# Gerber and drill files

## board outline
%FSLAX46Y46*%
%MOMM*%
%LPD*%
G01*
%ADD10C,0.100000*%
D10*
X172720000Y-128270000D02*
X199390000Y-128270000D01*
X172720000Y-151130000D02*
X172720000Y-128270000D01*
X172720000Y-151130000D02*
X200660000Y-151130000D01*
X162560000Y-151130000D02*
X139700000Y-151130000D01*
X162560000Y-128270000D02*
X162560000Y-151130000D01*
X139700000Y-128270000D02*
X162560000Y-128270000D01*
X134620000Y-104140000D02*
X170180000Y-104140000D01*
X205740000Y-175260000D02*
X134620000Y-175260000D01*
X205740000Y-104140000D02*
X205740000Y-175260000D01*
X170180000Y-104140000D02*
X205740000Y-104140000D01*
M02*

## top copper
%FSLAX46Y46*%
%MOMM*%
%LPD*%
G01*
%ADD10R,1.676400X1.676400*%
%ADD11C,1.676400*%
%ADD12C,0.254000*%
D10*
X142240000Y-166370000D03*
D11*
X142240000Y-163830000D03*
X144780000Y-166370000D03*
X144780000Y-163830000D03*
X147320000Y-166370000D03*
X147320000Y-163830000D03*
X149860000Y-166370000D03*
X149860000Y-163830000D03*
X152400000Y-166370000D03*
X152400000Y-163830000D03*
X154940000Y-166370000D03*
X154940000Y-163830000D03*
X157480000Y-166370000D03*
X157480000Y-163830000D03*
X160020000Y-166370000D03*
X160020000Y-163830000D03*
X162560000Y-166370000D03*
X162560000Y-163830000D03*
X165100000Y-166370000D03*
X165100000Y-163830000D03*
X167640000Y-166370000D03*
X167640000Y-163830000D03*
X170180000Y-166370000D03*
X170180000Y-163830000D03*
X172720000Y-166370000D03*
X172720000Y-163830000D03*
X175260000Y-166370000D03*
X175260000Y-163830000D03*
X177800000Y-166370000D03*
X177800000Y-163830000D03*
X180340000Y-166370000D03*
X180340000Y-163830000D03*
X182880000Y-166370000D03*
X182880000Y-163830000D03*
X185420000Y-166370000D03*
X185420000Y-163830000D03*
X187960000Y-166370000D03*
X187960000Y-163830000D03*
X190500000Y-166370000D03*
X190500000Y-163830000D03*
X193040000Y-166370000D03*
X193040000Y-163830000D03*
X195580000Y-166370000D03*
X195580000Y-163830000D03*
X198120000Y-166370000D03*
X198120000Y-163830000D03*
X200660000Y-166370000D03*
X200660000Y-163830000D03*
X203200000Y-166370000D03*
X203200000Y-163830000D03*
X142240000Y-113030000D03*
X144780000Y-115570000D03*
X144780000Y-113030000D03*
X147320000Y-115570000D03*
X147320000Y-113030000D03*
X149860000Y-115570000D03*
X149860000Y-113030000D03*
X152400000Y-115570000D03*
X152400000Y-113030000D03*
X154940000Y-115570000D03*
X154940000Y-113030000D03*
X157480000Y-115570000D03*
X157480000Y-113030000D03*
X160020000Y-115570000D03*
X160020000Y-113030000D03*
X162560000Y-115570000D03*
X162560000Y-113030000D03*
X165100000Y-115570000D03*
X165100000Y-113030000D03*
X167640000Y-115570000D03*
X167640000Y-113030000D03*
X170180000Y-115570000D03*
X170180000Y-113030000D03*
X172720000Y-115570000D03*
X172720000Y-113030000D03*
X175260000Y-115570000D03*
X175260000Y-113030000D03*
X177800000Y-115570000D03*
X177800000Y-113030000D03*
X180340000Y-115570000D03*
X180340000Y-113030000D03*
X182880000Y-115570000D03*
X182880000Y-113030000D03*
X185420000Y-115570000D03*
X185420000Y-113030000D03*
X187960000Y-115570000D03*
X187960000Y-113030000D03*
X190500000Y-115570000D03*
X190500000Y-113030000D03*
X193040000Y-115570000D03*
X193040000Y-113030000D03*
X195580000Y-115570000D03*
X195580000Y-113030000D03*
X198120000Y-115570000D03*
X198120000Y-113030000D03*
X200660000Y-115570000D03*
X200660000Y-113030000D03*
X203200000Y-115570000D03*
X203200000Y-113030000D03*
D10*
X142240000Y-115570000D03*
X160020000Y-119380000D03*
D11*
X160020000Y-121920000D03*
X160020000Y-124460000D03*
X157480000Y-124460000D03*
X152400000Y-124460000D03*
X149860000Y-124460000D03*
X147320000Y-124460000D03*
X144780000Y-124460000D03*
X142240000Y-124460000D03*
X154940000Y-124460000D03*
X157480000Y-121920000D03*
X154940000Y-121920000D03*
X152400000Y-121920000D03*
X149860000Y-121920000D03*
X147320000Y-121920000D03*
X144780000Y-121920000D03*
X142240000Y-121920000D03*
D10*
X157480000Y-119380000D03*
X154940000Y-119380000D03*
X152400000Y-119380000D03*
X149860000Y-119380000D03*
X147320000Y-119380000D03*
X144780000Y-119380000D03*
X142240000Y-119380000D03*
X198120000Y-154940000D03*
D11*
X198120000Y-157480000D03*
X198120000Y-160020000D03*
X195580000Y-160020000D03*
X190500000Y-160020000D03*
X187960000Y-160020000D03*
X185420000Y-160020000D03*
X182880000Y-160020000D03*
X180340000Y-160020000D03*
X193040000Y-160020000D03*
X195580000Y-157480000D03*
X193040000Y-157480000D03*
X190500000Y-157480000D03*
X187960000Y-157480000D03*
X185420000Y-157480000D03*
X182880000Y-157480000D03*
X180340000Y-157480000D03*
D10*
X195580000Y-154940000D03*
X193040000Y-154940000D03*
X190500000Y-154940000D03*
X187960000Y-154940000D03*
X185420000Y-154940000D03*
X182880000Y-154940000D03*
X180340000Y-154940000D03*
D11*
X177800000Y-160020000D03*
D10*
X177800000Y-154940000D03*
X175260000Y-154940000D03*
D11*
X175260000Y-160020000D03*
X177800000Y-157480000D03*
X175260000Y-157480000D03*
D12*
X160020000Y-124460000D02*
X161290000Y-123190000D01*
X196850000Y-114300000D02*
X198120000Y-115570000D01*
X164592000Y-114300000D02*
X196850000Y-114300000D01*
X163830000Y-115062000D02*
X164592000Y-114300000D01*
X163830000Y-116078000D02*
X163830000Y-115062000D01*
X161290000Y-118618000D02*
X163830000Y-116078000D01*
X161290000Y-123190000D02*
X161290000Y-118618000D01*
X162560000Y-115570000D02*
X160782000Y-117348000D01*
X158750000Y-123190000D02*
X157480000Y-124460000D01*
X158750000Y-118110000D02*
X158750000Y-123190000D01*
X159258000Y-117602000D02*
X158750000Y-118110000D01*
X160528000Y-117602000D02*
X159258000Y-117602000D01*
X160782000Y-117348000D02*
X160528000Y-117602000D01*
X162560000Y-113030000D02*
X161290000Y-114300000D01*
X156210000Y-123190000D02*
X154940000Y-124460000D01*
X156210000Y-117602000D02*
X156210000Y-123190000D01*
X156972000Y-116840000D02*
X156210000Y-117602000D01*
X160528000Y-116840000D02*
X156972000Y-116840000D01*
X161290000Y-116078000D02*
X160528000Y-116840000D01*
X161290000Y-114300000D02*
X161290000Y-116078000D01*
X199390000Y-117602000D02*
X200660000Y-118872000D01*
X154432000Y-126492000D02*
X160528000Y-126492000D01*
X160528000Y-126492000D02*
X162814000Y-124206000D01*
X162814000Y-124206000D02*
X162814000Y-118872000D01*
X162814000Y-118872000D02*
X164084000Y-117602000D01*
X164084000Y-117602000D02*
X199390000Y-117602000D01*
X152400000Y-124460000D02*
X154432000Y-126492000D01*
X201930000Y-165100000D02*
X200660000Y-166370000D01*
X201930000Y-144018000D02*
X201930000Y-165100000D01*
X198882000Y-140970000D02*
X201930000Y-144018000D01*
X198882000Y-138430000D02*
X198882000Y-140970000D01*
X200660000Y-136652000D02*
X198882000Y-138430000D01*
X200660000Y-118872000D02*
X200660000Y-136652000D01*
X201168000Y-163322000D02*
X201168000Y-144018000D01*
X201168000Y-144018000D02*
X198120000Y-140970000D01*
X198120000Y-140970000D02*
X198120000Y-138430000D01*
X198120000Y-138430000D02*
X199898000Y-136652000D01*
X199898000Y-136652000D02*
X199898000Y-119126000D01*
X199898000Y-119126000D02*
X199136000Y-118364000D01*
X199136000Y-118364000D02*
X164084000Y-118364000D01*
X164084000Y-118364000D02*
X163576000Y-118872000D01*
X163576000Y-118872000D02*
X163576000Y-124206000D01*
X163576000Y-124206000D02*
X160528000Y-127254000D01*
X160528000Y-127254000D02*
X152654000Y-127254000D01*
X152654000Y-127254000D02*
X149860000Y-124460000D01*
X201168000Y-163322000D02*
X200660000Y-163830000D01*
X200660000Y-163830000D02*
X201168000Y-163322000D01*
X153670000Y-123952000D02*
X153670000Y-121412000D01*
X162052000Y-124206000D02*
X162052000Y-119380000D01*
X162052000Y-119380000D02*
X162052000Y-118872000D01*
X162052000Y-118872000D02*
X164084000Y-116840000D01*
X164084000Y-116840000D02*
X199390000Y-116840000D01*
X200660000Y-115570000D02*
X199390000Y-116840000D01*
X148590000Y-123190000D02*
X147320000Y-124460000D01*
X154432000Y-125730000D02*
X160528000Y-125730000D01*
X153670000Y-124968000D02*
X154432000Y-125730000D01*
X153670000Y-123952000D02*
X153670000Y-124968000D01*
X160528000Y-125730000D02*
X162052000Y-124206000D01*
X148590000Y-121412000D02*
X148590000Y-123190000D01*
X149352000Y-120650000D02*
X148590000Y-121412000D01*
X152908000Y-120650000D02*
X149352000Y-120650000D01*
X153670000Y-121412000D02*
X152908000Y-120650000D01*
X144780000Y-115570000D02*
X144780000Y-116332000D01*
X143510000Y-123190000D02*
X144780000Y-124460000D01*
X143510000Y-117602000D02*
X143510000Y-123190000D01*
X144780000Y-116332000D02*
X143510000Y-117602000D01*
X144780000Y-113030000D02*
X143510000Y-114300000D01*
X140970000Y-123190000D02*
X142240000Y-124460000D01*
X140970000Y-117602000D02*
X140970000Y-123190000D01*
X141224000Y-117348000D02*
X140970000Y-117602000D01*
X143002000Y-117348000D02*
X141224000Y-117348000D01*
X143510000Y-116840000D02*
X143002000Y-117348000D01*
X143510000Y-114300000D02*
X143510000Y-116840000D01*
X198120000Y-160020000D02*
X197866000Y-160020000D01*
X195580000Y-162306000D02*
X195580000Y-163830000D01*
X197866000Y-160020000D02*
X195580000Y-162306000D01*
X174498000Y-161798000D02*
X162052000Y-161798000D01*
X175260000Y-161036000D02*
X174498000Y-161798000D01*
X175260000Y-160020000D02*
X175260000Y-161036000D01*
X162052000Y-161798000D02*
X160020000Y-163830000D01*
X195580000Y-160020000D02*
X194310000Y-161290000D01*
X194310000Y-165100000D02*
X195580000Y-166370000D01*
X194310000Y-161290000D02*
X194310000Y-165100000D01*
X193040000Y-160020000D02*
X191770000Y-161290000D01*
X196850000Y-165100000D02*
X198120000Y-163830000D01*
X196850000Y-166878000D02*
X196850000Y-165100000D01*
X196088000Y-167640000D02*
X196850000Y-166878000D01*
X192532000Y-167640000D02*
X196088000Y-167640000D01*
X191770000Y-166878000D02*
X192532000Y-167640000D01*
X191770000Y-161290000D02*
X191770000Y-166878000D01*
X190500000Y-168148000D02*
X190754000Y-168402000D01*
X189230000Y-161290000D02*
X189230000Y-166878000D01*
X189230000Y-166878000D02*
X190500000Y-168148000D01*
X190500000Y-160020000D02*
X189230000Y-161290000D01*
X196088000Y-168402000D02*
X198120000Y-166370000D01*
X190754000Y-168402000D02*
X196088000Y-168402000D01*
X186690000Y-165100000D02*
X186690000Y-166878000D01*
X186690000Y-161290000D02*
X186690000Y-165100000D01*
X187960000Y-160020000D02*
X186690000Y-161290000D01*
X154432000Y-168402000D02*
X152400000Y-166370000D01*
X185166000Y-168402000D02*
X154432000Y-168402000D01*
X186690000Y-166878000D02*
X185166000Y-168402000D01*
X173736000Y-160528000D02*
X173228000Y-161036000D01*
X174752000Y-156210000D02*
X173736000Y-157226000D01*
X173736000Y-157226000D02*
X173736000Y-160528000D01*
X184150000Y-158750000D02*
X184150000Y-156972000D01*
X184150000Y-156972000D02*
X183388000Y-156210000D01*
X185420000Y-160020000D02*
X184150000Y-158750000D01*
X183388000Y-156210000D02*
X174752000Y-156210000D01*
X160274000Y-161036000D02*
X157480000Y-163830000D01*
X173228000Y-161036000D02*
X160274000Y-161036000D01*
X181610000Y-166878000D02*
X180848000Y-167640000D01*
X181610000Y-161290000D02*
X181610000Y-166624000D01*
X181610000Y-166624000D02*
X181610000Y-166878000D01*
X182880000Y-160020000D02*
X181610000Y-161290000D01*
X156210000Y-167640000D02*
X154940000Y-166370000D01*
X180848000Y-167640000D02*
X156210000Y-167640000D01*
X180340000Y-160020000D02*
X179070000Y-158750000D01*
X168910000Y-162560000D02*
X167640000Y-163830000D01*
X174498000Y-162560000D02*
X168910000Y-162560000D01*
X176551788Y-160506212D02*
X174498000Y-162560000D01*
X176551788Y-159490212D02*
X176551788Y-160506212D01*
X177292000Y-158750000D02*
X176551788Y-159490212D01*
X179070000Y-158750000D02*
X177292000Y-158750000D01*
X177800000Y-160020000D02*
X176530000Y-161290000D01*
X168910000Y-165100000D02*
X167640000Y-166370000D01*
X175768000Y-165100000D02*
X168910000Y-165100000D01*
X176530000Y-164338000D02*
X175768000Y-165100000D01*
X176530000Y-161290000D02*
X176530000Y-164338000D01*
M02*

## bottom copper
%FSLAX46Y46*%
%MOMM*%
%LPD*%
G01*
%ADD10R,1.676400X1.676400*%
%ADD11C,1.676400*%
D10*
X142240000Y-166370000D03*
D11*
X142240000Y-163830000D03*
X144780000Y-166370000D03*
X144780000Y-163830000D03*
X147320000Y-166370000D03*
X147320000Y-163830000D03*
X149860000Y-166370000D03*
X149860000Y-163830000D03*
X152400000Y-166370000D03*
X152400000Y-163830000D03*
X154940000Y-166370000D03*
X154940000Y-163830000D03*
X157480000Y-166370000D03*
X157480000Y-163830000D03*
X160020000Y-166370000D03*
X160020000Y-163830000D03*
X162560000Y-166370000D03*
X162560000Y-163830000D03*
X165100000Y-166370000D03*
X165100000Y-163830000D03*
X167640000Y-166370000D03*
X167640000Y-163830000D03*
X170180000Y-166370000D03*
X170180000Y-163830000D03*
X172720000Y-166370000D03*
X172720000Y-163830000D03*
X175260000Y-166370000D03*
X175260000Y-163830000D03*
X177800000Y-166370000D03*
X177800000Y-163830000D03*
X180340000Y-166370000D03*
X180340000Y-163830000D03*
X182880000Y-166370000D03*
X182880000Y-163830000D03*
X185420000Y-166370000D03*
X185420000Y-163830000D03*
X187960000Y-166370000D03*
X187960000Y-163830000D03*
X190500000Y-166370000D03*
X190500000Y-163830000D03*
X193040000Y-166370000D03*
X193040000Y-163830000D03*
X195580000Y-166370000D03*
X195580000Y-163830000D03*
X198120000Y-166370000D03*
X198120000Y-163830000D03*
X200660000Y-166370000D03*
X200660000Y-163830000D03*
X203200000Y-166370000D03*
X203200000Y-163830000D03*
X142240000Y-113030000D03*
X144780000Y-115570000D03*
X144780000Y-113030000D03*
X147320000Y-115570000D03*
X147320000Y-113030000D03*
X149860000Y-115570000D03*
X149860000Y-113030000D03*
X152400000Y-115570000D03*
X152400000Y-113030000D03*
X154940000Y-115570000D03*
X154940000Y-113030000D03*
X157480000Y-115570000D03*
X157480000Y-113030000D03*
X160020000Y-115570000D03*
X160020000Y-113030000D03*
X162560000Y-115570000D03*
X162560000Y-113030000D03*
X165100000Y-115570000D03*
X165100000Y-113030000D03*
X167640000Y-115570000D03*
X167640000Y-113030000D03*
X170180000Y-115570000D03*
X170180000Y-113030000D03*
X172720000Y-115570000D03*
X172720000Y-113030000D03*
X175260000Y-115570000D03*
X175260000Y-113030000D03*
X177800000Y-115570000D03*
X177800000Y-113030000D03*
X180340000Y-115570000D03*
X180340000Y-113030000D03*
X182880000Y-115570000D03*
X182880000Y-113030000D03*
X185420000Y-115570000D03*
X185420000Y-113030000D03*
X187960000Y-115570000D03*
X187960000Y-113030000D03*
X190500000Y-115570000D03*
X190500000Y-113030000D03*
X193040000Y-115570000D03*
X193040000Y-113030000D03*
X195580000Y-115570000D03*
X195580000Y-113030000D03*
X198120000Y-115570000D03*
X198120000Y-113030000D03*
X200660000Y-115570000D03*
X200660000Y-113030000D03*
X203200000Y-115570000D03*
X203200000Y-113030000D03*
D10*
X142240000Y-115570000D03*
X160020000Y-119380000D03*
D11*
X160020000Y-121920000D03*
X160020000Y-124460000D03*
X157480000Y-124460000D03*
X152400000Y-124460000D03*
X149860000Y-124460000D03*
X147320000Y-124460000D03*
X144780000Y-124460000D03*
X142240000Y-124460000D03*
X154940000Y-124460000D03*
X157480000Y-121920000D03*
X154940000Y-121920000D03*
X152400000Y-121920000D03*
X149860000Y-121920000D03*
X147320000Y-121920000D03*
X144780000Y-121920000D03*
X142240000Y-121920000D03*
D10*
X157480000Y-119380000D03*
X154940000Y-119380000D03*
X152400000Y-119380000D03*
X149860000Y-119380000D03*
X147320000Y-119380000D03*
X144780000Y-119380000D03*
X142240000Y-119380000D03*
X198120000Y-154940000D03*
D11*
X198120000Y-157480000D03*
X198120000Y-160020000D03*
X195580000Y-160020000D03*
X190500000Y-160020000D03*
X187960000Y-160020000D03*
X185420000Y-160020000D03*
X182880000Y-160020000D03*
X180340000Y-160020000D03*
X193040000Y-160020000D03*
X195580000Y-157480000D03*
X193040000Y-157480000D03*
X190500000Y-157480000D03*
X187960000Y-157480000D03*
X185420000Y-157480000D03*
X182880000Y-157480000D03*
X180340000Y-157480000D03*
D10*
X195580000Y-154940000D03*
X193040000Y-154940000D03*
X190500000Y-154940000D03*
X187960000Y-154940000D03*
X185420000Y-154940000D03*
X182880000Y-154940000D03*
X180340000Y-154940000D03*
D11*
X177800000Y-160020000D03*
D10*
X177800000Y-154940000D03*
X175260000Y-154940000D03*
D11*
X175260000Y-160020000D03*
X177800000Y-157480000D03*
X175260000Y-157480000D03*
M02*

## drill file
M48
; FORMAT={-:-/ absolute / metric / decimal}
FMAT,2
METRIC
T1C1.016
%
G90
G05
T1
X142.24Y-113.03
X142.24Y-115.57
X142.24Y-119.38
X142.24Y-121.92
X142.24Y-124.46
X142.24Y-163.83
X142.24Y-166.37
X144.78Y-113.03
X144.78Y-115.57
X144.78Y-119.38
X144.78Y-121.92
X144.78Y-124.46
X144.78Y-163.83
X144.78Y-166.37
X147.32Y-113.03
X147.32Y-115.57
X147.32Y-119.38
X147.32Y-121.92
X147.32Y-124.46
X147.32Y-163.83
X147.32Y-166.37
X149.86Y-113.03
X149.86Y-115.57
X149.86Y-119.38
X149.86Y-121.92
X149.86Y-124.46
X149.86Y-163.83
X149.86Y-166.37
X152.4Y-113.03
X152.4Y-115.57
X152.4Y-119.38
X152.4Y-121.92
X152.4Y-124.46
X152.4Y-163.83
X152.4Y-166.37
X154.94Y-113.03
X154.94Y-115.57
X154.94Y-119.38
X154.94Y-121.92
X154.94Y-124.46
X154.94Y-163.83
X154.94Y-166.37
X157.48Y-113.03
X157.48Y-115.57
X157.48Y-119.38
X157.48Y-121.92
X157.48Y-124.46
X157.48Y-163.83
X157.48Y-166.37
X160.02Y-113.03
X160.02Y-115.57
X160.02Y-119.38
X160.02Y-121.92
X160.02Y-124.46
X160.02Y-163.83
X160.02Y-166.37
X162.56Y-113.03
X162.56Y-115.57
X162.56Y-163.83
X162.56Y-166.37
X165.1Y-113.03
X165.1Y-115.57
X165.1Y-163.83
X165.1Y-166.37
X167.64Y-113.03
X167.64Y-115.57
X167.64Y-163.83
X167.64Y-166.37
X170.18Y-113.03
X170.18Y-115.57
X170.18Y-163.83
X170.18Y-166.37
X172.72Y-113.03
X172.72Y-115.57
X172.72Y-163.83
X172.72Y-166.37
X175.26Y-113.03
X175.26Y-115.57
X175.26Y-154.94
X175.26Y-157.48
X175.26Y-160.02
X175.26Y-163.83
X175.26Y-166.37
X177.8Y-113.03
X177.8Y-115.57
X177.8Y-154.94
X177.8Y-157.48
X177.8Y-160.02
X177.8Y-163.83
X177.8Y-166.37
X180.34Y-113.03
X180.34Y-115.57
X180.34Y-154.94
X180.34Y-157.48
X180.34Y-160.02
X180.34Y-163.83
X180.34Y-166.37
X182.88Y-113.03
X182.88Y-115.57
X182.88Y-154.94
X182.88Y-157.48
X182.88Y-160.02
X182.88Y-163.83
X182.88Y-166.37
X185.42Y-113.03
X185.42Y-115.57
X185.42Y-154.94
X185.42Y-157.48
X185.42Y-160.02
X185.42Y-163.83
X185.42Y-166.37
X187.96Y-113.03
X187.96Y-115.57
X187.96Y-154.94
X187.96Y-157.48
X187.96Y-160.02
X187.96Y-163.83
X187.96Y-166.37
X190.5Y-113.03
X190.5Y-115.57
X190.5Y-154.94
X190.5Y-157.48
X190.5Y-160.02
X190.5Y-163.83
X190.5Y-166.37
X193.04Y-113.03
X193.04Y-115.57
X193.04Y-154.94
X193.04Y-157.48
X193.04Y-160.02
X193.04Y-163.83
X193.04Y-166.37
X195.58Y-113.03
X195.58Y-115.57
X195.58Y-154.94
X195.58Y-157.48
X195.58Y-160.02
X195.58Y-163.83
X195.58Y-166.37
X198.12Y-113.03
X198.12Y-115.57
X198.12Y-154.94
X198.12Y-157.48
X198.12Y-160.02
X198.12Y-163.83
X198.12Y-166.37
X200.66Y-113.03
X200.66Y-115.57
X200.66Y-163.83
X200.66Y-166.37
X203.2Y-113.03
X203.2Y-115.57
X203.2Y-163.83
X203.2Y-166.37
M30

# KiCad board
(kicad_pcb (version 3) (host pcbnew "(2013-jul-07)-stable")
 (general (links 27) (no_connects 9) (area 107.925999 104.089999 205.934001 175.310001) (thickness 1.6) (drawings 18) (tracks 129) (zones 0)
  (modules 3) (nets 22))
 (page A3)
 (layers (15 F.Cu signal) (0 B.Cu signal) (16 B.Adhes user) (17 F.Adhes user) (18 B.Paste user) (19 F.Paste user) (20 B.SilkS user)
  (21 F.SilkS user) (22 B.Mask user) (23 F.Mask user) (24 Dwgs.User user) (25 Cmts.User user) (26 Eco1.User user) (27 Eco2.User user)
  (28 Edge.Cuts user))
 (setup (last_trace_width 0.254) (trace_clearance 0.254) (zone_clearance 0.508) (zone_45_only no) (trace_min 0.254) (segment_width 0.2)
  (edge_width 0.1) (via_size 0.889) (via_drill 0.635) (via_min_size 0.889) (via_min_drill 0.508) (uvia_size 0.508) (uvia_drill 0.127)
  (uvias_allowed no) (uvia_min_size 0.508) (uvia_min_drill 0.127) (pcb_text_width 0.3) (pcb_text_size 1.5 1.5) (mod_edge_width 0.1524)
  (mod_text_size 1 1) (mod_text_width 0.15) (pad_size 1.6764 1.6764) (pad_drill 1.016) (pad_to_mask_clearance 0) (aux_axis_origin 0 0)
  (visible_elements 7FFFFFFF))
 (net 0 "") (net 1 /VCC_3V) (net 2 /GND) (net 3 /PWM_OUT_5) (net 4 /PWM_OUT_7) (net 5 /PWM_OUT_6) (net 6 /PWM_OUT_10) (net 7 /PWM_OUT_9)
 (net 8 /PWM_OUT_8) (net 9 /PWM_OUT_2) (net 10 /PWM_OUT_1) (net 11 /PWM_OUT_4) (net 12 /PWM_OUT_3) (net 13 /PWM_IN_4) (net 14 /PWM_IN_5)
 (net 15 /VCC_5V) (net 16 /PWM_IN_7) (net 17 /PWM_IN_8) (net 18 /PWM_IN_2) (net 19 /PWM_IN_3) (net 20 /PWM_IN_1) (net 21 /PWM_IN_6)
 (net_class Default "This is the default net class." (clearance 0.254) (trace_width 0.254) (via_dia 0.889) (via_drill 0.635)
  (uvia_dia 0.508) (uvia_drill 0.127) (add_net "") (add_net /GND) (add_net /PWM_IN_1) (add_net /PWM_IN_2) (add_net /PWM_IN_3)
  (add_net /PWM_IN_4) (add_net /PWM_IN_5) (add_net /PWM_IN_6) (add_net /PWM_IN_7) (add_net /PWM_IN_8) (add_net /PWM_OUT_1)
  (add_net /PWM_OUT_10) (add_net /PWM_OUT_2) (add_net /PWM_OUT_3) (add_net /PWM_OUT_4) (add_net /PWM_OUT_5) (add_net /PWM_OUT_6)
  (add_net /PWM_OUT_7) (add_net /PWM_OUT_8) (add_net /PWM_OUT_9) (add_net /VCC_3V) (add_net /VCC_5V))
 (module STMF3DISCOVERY (layer F.Cu) (at 172.72 139.7)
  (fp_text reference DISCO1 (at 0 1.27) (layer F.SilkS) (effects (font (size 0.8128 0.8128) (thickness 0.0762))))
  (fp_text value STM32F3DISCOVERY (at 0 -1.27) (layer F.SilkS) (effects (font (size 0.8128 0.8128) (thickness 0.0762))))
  (pad 6 thru_hole rect (at -30.48 26.67) (size 1.6764 1.6764) (drill 1.016) (layers *.Cu *.Mask F.SilkS) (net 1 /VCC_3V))
  (pad 20 thru_hole circle (at -30.48 24.13) (size 1.6764 1.6764) (drill 1.016) (layers *.Cu *.Mask F.SilkS) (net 1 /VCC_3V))
  (pad 49 thru_hole circle (at -27.94 26.67) (size 1.6764 1.6764) (drill 1.016) (layers *.Cu *.Mask F.SilkS) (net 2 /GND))
  (pad 14 thru_hole circle (at -27.94 24.13) (size 1.6764 1.6764) (drill 1.016) (layers *.Cu *.Mask F.SilkS))
  (pad 16 thru_hole circle (at -25.4 26.67) (size 1.6764 1.6764) (drill 1.016) (layers *.Cu *.Mask F.SilkS))
  (pad 15 thru_hole circle (at -25.4 24.13) (size 1.6764 1.6764) (drill 1.016) (layers *.Cu *.Mask F.SilkS))
  (pad 18 thru_hole circle (at -22.86 26.67) (size 1.6764 1.6764) (drill 1.016) (layers *.Cu *.Mask F.SilkS))
  (pad 17 thru_hole circle (at -22.86 24.13) (size 1.6764 1.6764) (drill 1.016) (layers *.Cu *.Mask F.SilkS))
  (pad 24 thru_hole circle (at -20.32 26.67) (size 1.6764 1.6764) (drill 1.016) (layers *.Cu *.Mask F.SilkS) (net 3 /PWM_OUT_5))
  (pad 19 thru_hole circle (at -20.32 24.13) (size 1.6764 1.6764) (drill 1.016) (layers *.Cu *.Mask F.SilkS))
  (pad 26 thru_hole circle (at -17.78 26.67) (size 1.6764 1.6764) (drill 1.016) (layers *.Cu *.Mask F.SilkS) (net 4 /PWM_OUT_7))
  (pad 23 thru_hole circle (at -17.78 24.13) (size 1.6764 1.6764) (drill 1.016) (layers *.Cu *.Mask F.SilkS))
  (pad 27 thru_hole circle (at -15.24 26.67) (size 1.6764 1.6764) (drill 1.016) (layers *.Cu *.Mask F.SilkS))
  (pad 25 thru_hole circle (at -15.24 24.13) (size 1.6764 1.6764) (drill 1.016) (layers *.Cu *.Mask F.SilkS) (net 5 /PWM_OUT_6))
  (pad 30 thru_hole circle (at -12.7 26.67) (size 1.6764 1.6764) (drill 1.016) (layers *.Cu *.Mask F.SilkS))
  (pad 29 thru_hole circle (at -12.7 24.13) (size 1.6764 1.6764) (drill 1.016) (layers *.Cu *.Mask F.SilkS) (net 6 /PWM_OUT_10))
  (pad 32 thru_hole circle (at -10.16 26.67) (size 1.6764 1.6764) (drill 1.016) (layers *.Cu *.Mask F.SilkS))
  (pad 31 thru_hole circle (at -10.16 24.13) (size 1.6764 1.6764) (drill 1.016) (layers *.Cu *.Mask F.SilkS))
  (pad 34 thru_hole circle (at -7.62 26.67) (size 1.6764 1.6764) (drill 1.016) (layers *.Cu *.Mask F.SilkS))
  (pad 33 thru_hole circle (at -7.62 24.13) (size 1.6764 1.6764) (drill 1.016) (layers *.Cu *.Mask F.SilkS))
  (pad 36 thru_hole circle (at -5.08 26.67) (size 1.6764 1.6764) (drill 1.016) (layers *.Cu *.Mask F.SilkS) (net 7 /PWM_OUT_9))
  (pad 35 thru_hole circle (at -5.08 24.13) (size 1.6764 1.6764) (drill 1.016) (layers *.Cu *.Mask F.SilkS) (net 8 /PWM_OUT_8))
  (pad 38 thru_hole circle (at -2.54 26.67) (size 1.6764 1.6764) (drill 1.016) (layers *.Cu *.Mask F.SilkS))
  (pad 37 thru_hole circle (at -2.54 24.13) (size 1.6764 1.6764) (drill 1.016) (layers *.Cu *.Mask F.SilkS))
  (pad 40 thru_hole circle (at 0 26.67) (size 1.6764 1.6764) (drill 1.016) (layers *.Cu *.Mask F.SilkS))
  (pad 39 thru_hole circle (at 0 24.13) (size 1.6764 1.6764) (drill 1.016) (layers *.Cu *.Mask F.SilkS))
  (pad 42 thru_hole circle (at 2.54 26.67) (size 1.6764 1.6764) (drill 1.016) (layers *.Cu *.Mask F.SilkS))
  (pad 41 thru_hole circle (at 2.54 24.13) (size 1.6764 1.6764) (drill 1.016) (layers *.Cu *.Mask F.SilkS))
  (pad 44 thru_hole circle (at 5.08 26.67) (size 1.6764 1.6764) (drill 1.016) (layers *.Cu *.Mask F.SilkS))
  (pad 43 thru_hole circle (at 5.08 24.13) (size 1.6764 1.6764) (drill 1.016) (layers *.Cu *.Mask F.SilkS))
  (pad 46 thru_hole circle (at 7.62 26.67) (size 1.6764 1.6764) (drill 1.016) (layers *.Cu *.Mask F.SilkS))
  (pad 45 thru_hole circle (at 7.62 24.13) (size 1.6764 1.6764) (drill 1.016) (layers *.Cu *.Mask F.SilkS))
  (pad 48 thru_hole circle (at 10.16 26.67) (size 1.6764 1.6764) (drill 1.016) (layers *.Cu *.Mask F.SilkS))
  (pad 47 thru_hole circle (at 10.16 24.13) (size 1.6764 1.6764) (drill 1.016) (layers *.Cu *.Mask F.SilkS))
  (pad 52 thru_hole circle (at 12.7 26.67) (size 1.6764 1.6764) (drill 1.016) (layers *.Cu *.Mask F.SilkS))
  (pad 51 thru_hole circle (at 12.7 24.13) (size 1.6764 1.6764) (drill 1.016) (layers *.Cu *.Mask F.SilkS))
  (pad 54 thru_hole circle (at 15.24 26.67) (size 1.6764 1.6764) (drill 1.016) (layers *.Cu *.Mask F.SilkS))
  (pad 53 thru_hole circle (at 15.24 24.13) (size 1.6764 1.6764) (drill 1.016) (layers *.Cu *.Mask F.SilkS))
  (pad 56 thru_hole circle (at 17.78 26.67) (size 1.6764 1.6764) (drill 1.016) (layers *.Cu *.Mask F.SilkS))
  (pad 55 thru_hole circle (at 17.78 24.13) (size 1.6764 1.6764) (drill 1.016) (layers *.Cu *.Mask F.SilkS))
  (pad 58 thru_hole circle (at 20.32 26.67) (size 1.6764 1.6764) (drill 1.016) (layers *.Cu *.Mask F.SilkS))
  (pad 57 thru_hole circle (at 20.32 24.13) (size 1.6764 1.6764) (drill 1.016) (layers *.Cu *.Mask F.SilkS))
  (pad 60 thru_hole circle (at 22.86 26.67) (size 1.6764 1.6764) (drill 1.016) (layers *.Cu *.Mask F.SilkS) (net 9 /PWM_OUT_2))
  (pad 59 thru_hole circle (at 22.86 24.13) (size 1.6764 1.6764) (drill 1.016) (layers *.Cu *.Mask F.SilkS) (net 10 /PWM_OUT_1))
  (pad 62 thru_hole circle (at 25.4 26.67) (size 1.6764 1.6764) (drill 1.016) (layers *.Cu *.Mask F.SilkS) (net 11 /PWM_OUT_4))
  (pad 61 thru_hole circle (at 25.4 24.13) (size 1.6764 1.6764) (drill 1.016) (layers *.Cu *.Mask F.SilkS) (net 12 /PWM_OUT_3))
  (pad 63 thru_hole circle (at 27.94 26.67) (size 1.6764 1.6764) (drill 1.016) (layers *.Cu *.Mask F.SilkS) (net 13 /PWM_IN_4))
  (pad 64 thru_hole circle (at 27.94 24.13) (size 1.6764 1.6764) (drill 1.016) (layers *.Cu *.Mask F.SilkS) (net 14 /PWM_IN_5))
  (pad 50 thru_hole circle (at 30.48 26.67) (size 1.6764 1.6764) (drill 1.016) (layers *.Cu *.Mask F.SilkS) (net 2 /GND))
  (pad 74 thru_hole circle (at 30.48 24.13) (size 1.6764 1.6764) (drill 1.016) (layers *.Cu *.Mask F.SilkS) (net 2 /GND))
  (pad 22 thru_hole circle (at -30.48 -26.67) (size 1.6764 1.6764) (drill 1.016) (layers *.Cu *.Mask F.SilkS) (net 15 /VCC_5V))
  (pad 10 thru_hole circle (at -27.94 -24.13) (size 1.6764 1.6764) (drill 1.016) (layers *.Cu *.Mask F.SilkS) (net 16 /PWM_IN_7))
  (pad 11 thru_hole circle (at -27.94 -26.67) (size 1.6764 1.6764) (drill 1.016) (layers *.Cu *.Mask F.SilkS) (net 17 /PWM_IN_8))
  (pad 12 thru_hole circle (at -25.4 -24.13) (size 1.6764 1.6764) (drill 1.016) (layers *.Cu *.Mask F.SilkS))
  (pad 13 thru_hole circle (at -25.4 -26.67) (size 1.6764 1.6764) (drill 1.016) (layers *.Cu *.Mask F.SilkS))
  (pad 8 thru_hole circle (at -22.86 -24.13) (size 1.6764 1.6764) (drill 1.016) (layers *.Cu *.Mask F.SilkS))
  (pad 9 thru_hole circle (at -22.86 -26.67) (size 1.6764 1.6764) (drill 1.016) (layers *.Cu *.Mask F.SilkS))
  (pad 5 thru_hole circle (at -20.32 -24.13) (size 1.6764 1.6764) (drill 1.016) (layers *.Cu *.Mask F.SilkS))
  (pad 7 thru_hole circle (at -20.32 -26.67) (size 1.6764 1.6764) (drill 1.016) (layers *.Cu *.Mask F.SilkS))
  (pad 3 thru_hole circle (at -17.78 -24.13) (size 1.6764 1.6764) (drill 1.016) (layers *.Cu *.Mask F.SilkS))
  (pad 4 thru_hole circle (at -17.78 -26.67) (size 1.6764 1.6764) (drill 1.016) (layers *.Cu *.Mask F.SilkS))
  (pad 1 thru_hole circle (at -15.24 -24.13) (size 1.6764 1.6764) (drill 1.016) (layers *.Cu *.Mask F.SilkS))
  (pad 2 thru_hole circle (at -15.24 -26.67) (size 1.6764 1.6764) (drill 1.016) (layers *.Cu *.Mask F.SilkS))
  (pad 97 thru_hole circle (at -12.7 -24.13) (size 1.6764 1.6764) (drill 1.016) (layers *.Cu *.Mask F.SilkS))
  (pad 98 thru_hole circle (at -12.7 -26.67) (size 1.6764 1.6764) (drill 1.016) (layers *.Cu *.Mask F.SilkS))
  (pad 95 thru_hole circle (at -10.16 -24.13) (size 1.6764 1.6764) (drill 1.016) (layers *.Cu *.Mask F.SilkS) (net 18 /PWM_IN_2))
  (pad 96 thru_hole circle (at -10.16 -26.67) (size 1.6764 1.6764) (drill 1.016) (layers *.Cu *.Mask F.SilkS) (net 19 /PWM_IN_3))
  (pad 94 thru_hole circle (at -7.62 -24.13) (size 1.6764 1.6764) (drill 1.016) (layers *.Cu *.Mask F.SilkS))
  (pad 28 thru_hole circle (at -7.62 -26.67) (size 1.6764 1.6764) (drill 1.016) (layers *.Cu *.Mask F.SilkS))
  (pad 92 thru_hole circle (at -5.08 -24.13) (size 1.6764 1.6764) (drill 1.016) (layers *.Cu *.Mask F.SilkS))
  (pad 93 thru_hole circle (at -5.08 -26.67) (size 1.6764 1.6764) (drill 1.016) (layers *.Cu *.Mask F.SilkS))
  (pad 90 thru_hole circle (at -2.54 -24.13) (size 1.6764 1.6764) (drill 1.016) (layers *.Cu *.Mask F.SilkS))
  (pad 91 thru_hole circle (at -2.54 -26.67) (size 1.6764 1.6764) (drill 1.016) (layers *.Cu *.Mask F.SilkS))
  (pad 88 thru_hole circle (at 0 -24.13) (size 1.6764 1.6764) (drill 1.016) (layers *.Cu *.Mask F.SilkS))
  (pad 89 thru_hole circle (at 0 -26.67) (size 1.6764 1.6764) (drill 1.016) (layers *.Cu *.Mask F.SilkS))
  (pad 86 thru_hole circle (at 2.54 -24.13) (size 1.6764 1.6764) (drill 1.016) (layers *.Cu *.Mask F.SilkS))
  (pad 87 thru_hole circle (at 2.54 -26.67) (size 1.6764 1.6764) (drill 1.016) (layers *.Cu *.Mask F.SilkS))
  (pad 84 thru_hole circle (at 5.08 -24.13) (size 1.6764 1.6764) (drill 1.016) (layers *.Cu *.Mask F.SilkS))
  (pad 85 thru_hole circle (at 5.08 -26.67) (size 1.6764 1.6764) (drill 1.016) (layers *.Cu *.Mask F.SilkS))
  (pad 82 thru_hole circle (at 7.62 -24.13) (size 1.6764 1.6764) (drill 1.016) (layers *.Cu *.Mask F.SilkS))
  (pad 83 thru_hole circle (at 7.62 -26.67) (size 1.6764 1.6764) (drill 1.016) (layers *.Cu *.Mask F.SilkS))
  (pad 80 thru_hole circle (at 10.16 -24.13) (size 1.6764 1.6764) (drill 1.016) (layers *.Cu *.Mask F.SilkS))
  (pad 81 thru_hole circle (at 10.16 -26.67) (size 1.6764 1.6764) (drill 1.016) (layers *.Cu *.Mask F.SilkS))
  (pad 78 thru_hole circle (at 12.7 -24.13) (size 1.6764 1.6764) (drill 1.016) (layers *.Cu *.Mask F.SilkS))
  (pad 79 thru_hole circle (at 12.7 -26.67) (size 1.6764 1.6764) (drill 1.016) (layers *.Cu *.Mask F.SilkS))
  (pad 76 thru_hole circle (at 15.24 -24.13) (size 1.6764 1.6764) (drill 1.016) (layers *.Cu *.Mask F.SilkS))
  (pad 77 thru_hole circle (at 15.24 -26.67) (size 1.6764 1.6764) (drill 1.016) (layers *.Cu *.Mask F.SilkS))
  (pad 73 thru_hole circle (at 17.78 -24.13) (size 1.6764 1.6764) (drill 1.016) (layers *.Cu *.Mask F.SilkS))
  (pad 72 thru_hole circle (at 17.78 -26.67) (size 1.6764 1.6764) (drill 1.016) (layers *.Cu *.Mask F.SilkS))
  (pad 71 thru_hole circle (at 20.32 -24.13) (size 1.6764 1.6764) (drill 1.016) (layers *.Cu *.Mask F.SilkS))
  (pad 70 thru_hole circle (at 20.32 -26.67) (size 1.6764 1.6764) (drill 1.016) (layers *.Cu *.Mask F.SilkS))
  (pad 69 thru_hole circle (at 22.86 -24.13) (size 1.6764 1.6764) (drill 1.016) (layers *.Cu *.Mask F.SilkS))
  (pad 68 thru_hole circle (at 22.86 -26.67) (size 1.6764 1.6764) (drill 1.016) (layers *.Cu *.Mask F.SilkS))
  (pad 67 thru_hole circle (at 25.4 -24.13) (size 1.6764 1.6764) (drill 1.016) (layers *.Cu *.Mask F.SilkS) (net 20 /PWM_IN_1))
  (pad 66 thru_hole circle (at 25.4 -26.67) (size 1.6764 1.6764) (drill 1.016) (layers *.Cu *.Mask F.SilkS))
  (pad 65 thru_hole circle (at 27.94 -24.13) (size 1.6764 1.6764) (drill 1.016) (layers *.Cu *.Mask F.SilkS) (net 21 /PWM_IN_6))
  (pad 100 thru_hole circle (at 27.94 -26.67) (size 1.6764 1.6764) (drill 1.016) (layers *.Cu *.Mask F.SilkS))
  (pad 75 thru_hole circle (at 30.48 -24.13) (size 1.6764 1.6764) (drill 1.016) (layers *.Cu *.Mask F.SilkS) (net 2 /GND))
  (pad 99 thru_hole circle (at 30.48 -26.67) (size 1.6764 1.6764) (drill 1.016) (layers *.Cu *.Mask F.SilkS) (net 2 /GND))
  (pad 21 thru_hole rect (at -30.48 -24.13) (size 1.6764 1.6764) (drill 1.016) (layers *.Cu *.Mask F.SilkS) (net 15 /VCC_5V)))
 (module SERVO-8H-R (layer F.Cu) (at 151.13 121.92 180)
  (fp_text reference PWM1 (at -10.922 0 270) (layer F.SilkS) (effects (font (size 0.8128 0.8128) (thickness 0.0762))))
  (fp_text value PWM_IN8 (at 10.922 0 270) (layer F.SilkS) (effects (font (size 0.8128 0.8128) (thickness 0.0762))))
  (pad 1 thru_hole rect (at -8.89 2.54 180) (size 1.6764 1.6764) (drill 1.016) (layers *.Cu *.Mask F.SilkS) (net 2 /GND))
  (pad 2 thru_hole circle (at -8.89 0 180) (size 1.6764 1.6764) (drill 1.016) (layers *.Cu *.Mask F.SilkS))
  (pad 3 thru_hole circle (at -8.89 -2.54 180) (size 1.6764 1.6764) (drill 1.016) (layers *.Cu *.Mask F.SilkS) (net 20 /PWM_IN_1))
  (pad 4 thru_hole circle (at -6.35 -2.54 180) (size 1.6764 1.6764) (drill 1.016) (layers *.Cu *.Mask F.SilkS) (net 18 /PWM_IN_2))
  (pad 6 thru_hole circle (at -1.27 -2.54 180) (size 1.6764 1.6764) (drill 1.016) (layers *.Cu *.Mask F.SilkS) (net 13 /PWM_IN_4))
  (pad 7 thru_hole circle (at 1.27 -2.54 180) (size 1.6764 1.6764) (drill 1.016) (layers *.Cu *.Mask F.SilkS) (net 14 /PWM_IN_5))
  (pad 8 thru_hole circle (at 3.81 -2.54 180) (size 1.6764 1.6764) (drill 1.016) (layers *.Cu *.Mask F.SilkS) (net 21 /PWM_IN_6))
  (pad 9 thru_hole circle (at 6.35 -2.54 180) (size 1.6764 1.6764) (drill 1.016) (layers *.Cu *.Mask F.SilkS) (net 16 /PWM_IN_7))
  (pad 10 thru_hole circle (at 8.89 -2.54 180) (size 1.6764 1.6764) (drill 1.016) (layers *.Cu *.Mask F.SilkS) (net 17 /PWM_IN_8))
  (pad 5 thru_hole circle (at -3.81 -2.54 180) (size 1.6764 1.6764) (drill 1.016) (layers *.Cu *.Mask F.SilkS) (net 19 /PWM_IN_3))
  (pad "" thru_hole circle (at -6.35 0 180) (size 1.6764 1.6764) (drill 1.016) (layers *.Cu *.Mask F.SilkS))
  (pad "" thru_hole circle (at -3.81 0 180) (size 1.6764 1.6764) (drill 1.016) (layers *.Cu *.Mask F.SilkS))
  (pad "" thru_hole circle (at -1.27 0 180) (size 1.6764 1.6764) (drill 1.016) (layers *.Cu *.Mask F.SilkS))
  (pad "" thru_hole circle (at 1.27 0 180) (size 1.6764 1.6764) (drill 1.016) (layers *.Cu *.Mask F.SilkS))
  (pad "" thru_hole circle (at 3.81 0 180) (size 1.6764 1.6764) (drill 1.016) (layers *.Cu *.Mask F.SilkS))
  (pad "" thru_hole circle (at 6.35 0 180) (size 1.6764 1.6764) (drill 1.016) (layers *.Cu *.Mask F.SilkS))
  (pad "" thru_hole circle (at 8.89 0 180) (size 1.6764 1.6764) (drill 1.016) (layers *.Cu *.Mask F.SilkS))
  (pad "" thru_hole rect (at -6.35 2.54 180) (size 1.6764 1.6764) (drill 1.016) (layers *.Cu *.Mask F.SilkS))
  (pad "" thru_hole rect (at -3.81 2.54 180) (size 1.6764 1.6764) (drill 1.016) (layers *.Cu *.Mask F.SilkS))
  (pad "" thru_hole rect (at -1.27 2.54 180) (size 1.6764 1.6764) (drill 1.016) (layers *.Cu *.Mask F.SilkS))
  (pad "" thru_hole rect (at 1.27 2.54 180) (size 1.6764 1.6764) (drill 1.016) (layers *.Cu *.Mask F.SilkS))
  (pad "" thru_hole rect (at 3.81 2.54 180) (size 1.6764 1.6764) (drill 1.016) (layers *.Cu *.Mask F.SilkS))
  (pad "" thru_hole rect (at 6.35 2.54 180) (size 1.6764 1.6764) (drill 1.016) (layers *.Cu *.Mask F.SilkS))
  (pad "" thru_hole rect (at 8.89 2.54 180) (size 1.6764 1.6764) (drill 1.016) (layers *.Cu *.Mask F.SilkS)))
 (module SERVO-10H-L (layer F.Cu) (at 186.69 157.48 180)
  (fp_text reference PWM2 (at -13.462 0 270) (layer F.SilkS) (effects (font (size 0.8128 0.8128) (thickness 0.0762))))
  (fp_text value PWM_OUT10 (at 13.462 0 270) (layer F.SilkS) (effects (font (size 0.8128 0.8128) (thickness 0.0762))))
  (pad 1 thru_hole rect (at -11.43 2.54 180) (size 1.6764 1.6764) (drill 1.016) (layers *.Cu *.Mask F.SilkS) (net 2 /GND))
  (pad 2 thru_hole circle (at -11.43 0 180) (size 1.6764 1.6764) (drill 1.016) (layers *.Cu *.Mask F.SilkS))
  (pad 3 thru_hole circle (at -11.43 -2.54 180) (size 1.6764 1.6764) (drill 1.016) (layers *.Cu *.Mask F.SilkS) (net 10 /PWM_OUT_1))
  (pad 4 thru_hole circle (at -8.89 -2.54 180) (size 1.6764 1.6764) (drill 1.016) (layers *.Cu *.Mask F.SilkS) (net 9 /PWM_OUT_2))
  (pad 6 thru_hole circle (at -3.81 -2.54 180) (size 1.6764 1.6764) (drill 1.016) (layers *.Cu *.Mask F.SilkS) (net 11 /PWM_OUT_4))
  (pad 7 thru_hole circle (at -1.27 -2.54 180) (size 1.6764 1.6764) (drill 1.016) (layers *.Cu *.Mask F.SilkS) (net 3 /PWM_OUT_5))
  (pad 8 thru_hole circle (at 1.27 -2.54 180) (size 1.6764 1.6764) (drill 1.016) (layers *.Cu *.Mask F.SilkS) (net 5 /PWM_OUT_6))
  (pad 9 thru_hole circle (at 3.81 -2.54 180) (size 1.6764 1.6764) (drill 1.016) (layers *.Cu *.Mask F.SilkS) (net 4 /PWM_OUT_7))
  (pad 10 thru_hole circle (at 6.35 -2.54 180) (size 1.6764 1.6764) (drill 1.016) (layers *.Cu *.Mask F.SilkS) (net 8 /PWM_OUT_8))
  (pad 5 thru_hole circle (at -6.35 -2.54 180) (size 1.6764 1.6764) (drill 1.016) (layers *.Cu *.Mask F.SilkS) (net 12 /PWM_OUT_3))
  (pad "" thru_hole circle (at -8.89 0 180) (size 1.6764 1.6764) (drill 1.016) (layers *.Cu *.Mask F.SilkS))
  (pad "" thru_hole circle (at -6.35 0 180) (size 1.6764 1.6764) (drill 1.016) (layers *.Cu *.Mask F.SilkS))
  (pad "" thru_hole circle (at -3.81 0 180) (size 1.6764 1.6764) (drill 1.016) (layers *.Cu *.Mask F.SilkS))
  (pad "" thru_hole circle (at -1.27 0 180) (size 1.6764 1.6764) (drill 1.016) (layers *.Cu *.Mask F.SilkS))
  (pad "" thru_hole circle (at 1.27 0 180) (size 1.6764 1.6764) (drill 1.016) (layers *.Cu *.Mask F.SilkS))
  (pad "" thru_hole circle (at 3.81 0 180) (size 1.6764 1.6764) (drill 1.016) (layers *.Cu *.Mask F.SilkS))
  (pad "" thru_hole circle (at 6.35 0 180) (size 1.6764 1.6764) (drill 1.016) (layers *.Cu *.Mask F.SilkS))
  (pad "" thru_hole rect (at -8.89 2.54 180) (size 1.6764 1.6764) (drill 1.016) (layers *.Cu *.Mask F.SilkS))
  (pad "" thru_hole rect (at -6.35 2.54 180) (size 1.6764 1.6764) (drill 1.016) (layers *.Cu *.Mask F.SilkS))
  (pad "" thru_hole rect (at -3.81 2.54 180) (size 1.6764 1.6764) (drill 1.016) (layers *.Cu *.Mask F.SilkS))
  (pad "" thru_hole rect (at -1.27 2.54 180) (size 1.6764 1.6764) (drill 1.016) (layers *.Cu *.Mask F.SilkS))
  (pad "" thru_hole rect (at 1.27 2.54 180) (size 1.6764 1.6764) (drill 1.016) (layers *.Cu *.Mask F.SilkS))
  (pad "" thru_hole rect (at 3.81 2.54 180) (size 1.6764 1.6764) (drill 1.016) (layers *.Cu *.Mask F.SilkS))
  (pad "" thru_hole rect (at 6.35 2.54 180) (size 1.6764 1.6764) (drill 1.016) (layers *.Cu *.Mask F.SilkS))
  (pad 11 thru_hole circle (at 8.89 -2.54 180) (size 1.6764 1.6764) (drill 1.016) (layers *.Cu *.Mask F.SilkS) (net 7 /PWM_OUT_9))
  (pad "" thru_hole rect (at 8.89 2.54 180) (size 1.6764 1.6764) (drill 1.016) (layers *.Cu *.Mask F.SilkS))
  (pad "" thru_hole rect (at 11.43 2.54 180) (size 1.6764 1.6764) (drill 1.016) (layers *.Cu *.Mask F.SilkS))
  (pad 12 thru_hole circle (at 11.43 -2.54 180) (size 1.6764 1.6764) (drill 1.016) (layers *.Cu *.Mask F.SilkS) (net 6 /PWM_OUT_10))
  (pad "" thru_hole circle (at 8.89 0 180) (size 1.6764 1.6764) (drill 1.016) (layers *.Cu *.Mask F.SilkS))
  (pad "" thru_hole circle (at 11.43 0 180) (size 1.6764 1.6764) (drill 1.016) (layers *.Cu *.Mask F.SilkS)))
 (gr_line (start 172.72 128.27) (end 199.39 128.27) (angle 90) (layer Edge.Cuts) (width 0.1))
 (gr_line (start 172.72 151.13) (end 172.72 128.27) (angle 90) (layer Edge.Cuts) (width 0.1))
 (gr_line (start 172.72 151.13) (end 200.66 151.13) (angle 90) (layer Edge.Cuts) (width 0.1))
 (gr_line (start 162.56 151.13) (end 139.7 151.13) (angle 90) (layer Edge.Cuts) (width 0.1))
 (gr_line (start 162.56 128.27) (end 162.56 151.13) (angle 90) (layer Edge.Cuts) (width 0.1))
 (gr_line (start 139.7 128.27) (end 162.56 128.27) (angle 90) (layer Edge.Cuts) (width 0.1))
 (gr_line (start 134.62 104.14) (end 170.18 104.14) (angle 90) (layer Edge.Cuts) (width 0.1))
 (gr_line (start 205.74 175.26) (end 134.62 175.26) (angle 90) (layer Edge.Cuts) (width 0.1))
 (gr_line (start 205.74 104.14) (end 205.74 175.26) (angle 90) (layer Edge.Cuts) (width 0.1))
 (gr_line (start 170.18 104.14) (end 205.74 104.14) (angle 90) (layer Edge.Cuts) (width 0.1))
 (segment (start 160.02 124.46) (end 161.29 123.19) (width 0.254) (layer F.Cu) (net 20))
 (segment (start 196.85 114.3) (end 198.12 115.57) (width 0.254) (layer F.Cu) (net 20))
 (segment (start 164.592 114.3) (end 196.85 114.3) (width 0.254) (layer F.Cu) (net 20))
 (segment (start 163.83 115.062) (end 164.592 114.3) (width 0.254) (layer F.Cu) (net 20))
 (segment (start 163.83 116.078) (end 163.83 115.062) (width 0.254) (layer F.Cu) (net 20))
 (segment (start 161.29 118.618) (end 163.83 116.078) (width 0.254) (layer F.Cu) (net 20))
 (segment (start 161.29 123.19) (end 161.29 118.618) (width 0.254) (layer F.Cu) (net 20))
 (segment (start 162.56 115.57) (end 160.782 117.348) (width 0.254) (layer F.Cu) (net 18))
 (segment (start 158.75 123.19) (end 157.48 124.46) (width 0.254) (layer F.Cu) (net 18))
 (segment (start 158.75 118.11) (end 158.75 123.19) (width 0.254) (layer F.Cu) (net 18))
 (segment (start 159.258 117.602) (end 158.75 118.11) (width 0.254) (layer F.Cu) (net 18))
 (segment (start 160.528 117.602) (end 159.258 117.602) (width 0.254) (layer F.Cu) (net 18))
 (segment (start 160.782 117.348) (end 160.528 117.602) (width 0.254) (layer F.Cu) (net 18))
 (segment (start 162.56 113.03) (end 161.29 114.3) (width 0.254) (layer F.Cu) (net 19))
 (segment (start 156.21 123.19) (end 154.94 124.46) (width 0.254) (layer F.Cu) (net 19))
 (segment (start 156.21 117.602) (end 156.21 123.19) (width 0.254) (layer F.Cu) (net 19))
 (segment (start 156.972 116.84) (end 156.21 117.602) (width 0.254) (layer F.Cu) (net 19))
 (segment (start 160.528 116.84) (end 156.972 116.84) (width 0.254) (layer F.Cu) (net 19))
 (segment (start 161.29 116.078) (end 160.528 116.84) (width 0.254) (layer F.Cu) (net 19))
 (segment (start 161.29 114.3) (end 161.29 116.078) (width 0.254) (layer F.Cu) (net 19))
 (segment (start 199.39 117.602) (end 200.66 118.872) (width 0.254) (layer F.Cu) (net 13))
 (segment (start 154.432 126.492) (end 160.528 126.492) (width 0.254) (layer F.Cu) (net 13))
 (segment (start 160.528 126.492) (end 162.814 124.206) (width 0.254) (layer F.Cu) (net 13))
 (segment (start 162.814 124.206) (end 162.814 118.872) (width 0.254) (layer F.Cu) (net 13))
 (segment (start 162.814 118.872) (end 164.084 117.602) (width 0.254) (layer F.Cu) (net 13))
 (segment (start 164.084 117.602) (end 199.39 117.602) (width 0.254) (layer F.Cu) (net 13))
 (segment (start 152.4 124.46) (end 154.432 126.492) (width 0.254) (layer F.Cu) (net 13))
 (segment (start 201.93 165.1) (end 200.66 166.37) (width 0.254) (layer F.Cu) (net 13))
 (segment (start 201.93 144.018) (end 201.93 165.1) (width 0.254) (layer F.Cu) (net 13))
 (segment (start 198.882 140.97) (end 201.93 144.018) (width 0.254) (layer F.Cu) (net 13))
 (segment (start 198.882 138.43) (end 198.882 140.97) (width 0.254) (layer F.Cu) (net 13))
 (segment (start 200.66 136.652) (end 198.882 138.43) (width 0.254) (layer F.Cu) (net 13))
 (segment (start 200.66 118.872) (end 200.66 136.652) (width 0.254) (layer F.Cu) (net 13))
 (segment (start 201.168 163.322) (end 201.168 144.018) (width 0.254) (layer F.Cu) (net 14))
 (segment (start 201.168 144.018) (end 198.12 140.97) (width 0.254) (layer F.Cu) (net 14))
 (segment (start 198.12 140.97) (end 198.12 138.43) (width 0.254) (layer F.Cu) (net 14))
 (segment (start 198.12 138.43) (end 199.898 136.652) (width 0.254) (layer F.Cu) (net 14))
 (segment (start 199.898 136.652) (end 199.898 119.126) (width 0.254) (layer F.Cu) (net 14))
 (segment (start 199.898 119.126) (end 199.136 118.364) (width 0.254) (layer F.Cu) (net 14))
 (segment (start 199.136 118.364) (end 164.084 118.364) (width 0.254) (layer F.Cu) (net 14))
 (segment (start 164.084 118.364) (end 163.576 118.872) (width 0.254) (layer F.Cu) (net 14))
 (segment (start 163.576 118.872) (end 163.576 124.206) (width 0.254) (layer F.Cu) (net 14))
 (segment (start 163.576 124.206) (end 160.528 127.254) (width 0.254) (layer F.Cu) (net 14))
 (segment (start 160.528 127.254) (end 152.654 127.254) (width 0.254) (layer F.Cu) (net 14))
 (segment (start 152.654 127.254) (end 149.86 124.46) (width 0.254) (layer F.Cu) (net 14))
 (segment (start 201.168 163.322) (end 200.66 163.83) (width 0.254) (layer F.Cu) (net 14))
 (segment (start 200.66 163.83) (end 201.168 163.322) (width 0.254) (layer F.Cu) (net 14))
 (segment (start 153.67 123.952) (end 153.67 121.412) (width 0.254) (layer F.Cu) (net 21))
 (segment (start 162.052 124.206) (end 162.052 119.38) (width 0.254) (layer F.Cu) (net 21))
 (segment (start 162.052 119.38) (end 162.052 118.872) (width 0.254) (layer F.Cu) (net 21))
 (segment (start 162.052 118.872) (end 164.084 116.84) (width 0.254) (layer F.Cu) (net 21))
 (segment (start 164.084 116.84) (end 199.39 116.84) (width 0.254) (layer F.Cu) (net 21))
 (segment (start 200.66 115.57) (end 199.39 116.84) (width 0.254) (layer F.Cu) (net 21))
 (segment (start 148.59 123.19) (end 147.32 124.46) (width 0.254) (layer F.Cu) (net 21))
 (segment (start 154.432 125.73) (end 160.528 125.73) (width 0.254) (layer F.Cu) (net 21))
 (segment (start 153.67 124.968) (end 154.432 125.73) (width 0.254) (layer F.Cu) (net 21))
 (segment (start 153.67 123.952) (end 153.67 124.968) (width 0.254) (layer F.Cu) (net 21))
 (segment (start 160.528 125.73) (end 162.052 124.206) (width 0.254) (layer F.Cu) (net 21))
 (segment (start 148.59 121.412) (end 148.59 123.19) (width 0.254) (layer F.Cu) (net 21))
 (segment (start 149.352 120.65) (end 148.59 121.412) (width 0.254) (layer F.Cu) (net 21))
 (segment (start 152.908 120.65) (end 149.352 120.65) (width 0.254) (layer F.Cu) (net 21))
 (segment (start 153.67 121.412) (end 152.908 120.65) (width 0.254) (layer F.Cu) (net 21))
 (segment (start 144.78 115.57) (end 144.78 116.332) (width 0.254) (layer F.Cu) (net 16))
 (segment (start 143.51 123.19) (end 144.78 124.46) (width 0.254) (layer F.Cu) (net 16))
 (segment (start 143.51 117.602) (end 143.51 123.19) (width 0.254) (layer F.Cu) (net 16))
 (segment (start 144.78 116.332) (end 143.51 117.602) (width 0.254) (layer F.Cu) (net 16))
 (segment (start 144.78 113.03) (end 143.51 114.3) (width 0.254) (layer F.Cu) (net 17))
 (segment (start 140.97 123.19) (end 142.24 124.46) (width 0.254) (layer F.Cu) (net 17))
 (segment (start 140.97 117.602) (end 140.97 123.19) (width 0.254) (layer F.Cu) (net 17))
 (segment (start 141.224 117.348) (end 140.97 117.602) (width 0.254) (layer F.Cu) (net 17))
 (segment (start 143.002 117.348) (end 141.224 117.348) (width 0.254) (layer F.Cu) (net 17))
 (segment (start 143.51 116.84) (end 143.002 117.348) (width 0.254) (layer F.Cu) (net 17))
 (segment (start 143.51 114.3) (end 143.51 116.84) (width 0.254) (layer F.Cu) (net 17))
 (segment (start 198.12 160.02) (end 197.866 160.02) (width 0.254) (layer F.Cu) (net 10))
 (segment (start 195.58 162.306) (end 195.58 163.83) (width 0.254) (layer F.Cu) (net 10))
 (segment (start 197.866 160.02) (end 195.58 162.306) (width 0.254) (layer F.Cu) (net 10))
 (segment (start 174.498 161.798) (end 162.052 161.798) (width 0.254) (layer F.Cu) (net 6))
 (segment (start 175.26 161.036) (end 174.498 161.798) (width 0.254) (layer F.Cu) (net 6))
 (segment (start 175.26 160.02) (end 175.26 161.036) (width 0.254) (layer F.Cu) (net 6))
 (segment (start 162.052 161.798) (end 160.02 163.83) (width 0.254) (layer F.Cu) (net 6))
 (segment (start 195.58 160.02) (end 194.31 161.29) (width 0.254) (layer F.Cu) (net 9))
 (segment (start 194.31 165.1) (end 195.58 166.37) (width 0.254) (layer F.Cu) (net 9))
 (segment (start 194.31 161.29) (end 194.31 165.1) (width 0.254) (layer F.Cu) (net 9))
 (segment (start 193.04 160.02) (end 191.77 161.29) (width 0.254) (layer F.Cu) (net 12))
 (segment (start 196.85 165.1) (end 198.12 163.83) (width 0.254) (layer F.Cu) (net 12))
 (segment (start 196.85 166.878) (end 196.85 165.1) (width 0.254) (layer F.Cu) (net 12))
 (segment (start 196.088 167.64) (end 196.85 166.878) (width 0.254) (layer F.Cu) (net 12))
 (segment (start 192.532 167.64) (end 196.088 167.64) (width 0.254) (layer F.Cu) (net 12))
 (segment (start 191.77 166.878) (end 192.532 167.64) (width 0.254) (layer F.Cu) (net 12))
 (segment (start 191.77 161.29) (end 191.77 166.878) (width 0.254) (layer F.Cu) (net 12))
 (segment (start 190.5 168.148) (end 190.754 168.402) (width 0.254) (layer F.Cu) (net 11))
 (segment (start 189.23 161.29) (end 189.23 166.878) (width 0.254) (layer F.Cu) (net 11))
 (segment (start 189.23 166.878) (end 190.5 168.148) (width 0.254) (layer F.Cu) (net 11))
 (segment (start 190.5 160.02) (end 189.23 161.29) (width 0.254) (layer F.Cu) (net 11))
 (segment (start 196.088 168.402) (end 198.12 166.37) (width 0.254) (layer F.Cu) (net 11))
 (segment (start 190.754 168.402) (end 196.088 168.402) (width 0.254) (layer F.Cu) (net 11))
 (segment (start 186.69 165.1) (end 186.69 166.878) (width 0.254) (layer F.Cu) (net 3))
 (segment (start 186.69 161.29) (end 186.69 165.1) (width 0.254) (layer F.Cu) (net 3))
 (segment (start 187.96 160.02) (end 186.69 161.29) (width 0.254) (layer F.Cu) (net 3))
 (segment (start 154.432 168.402) (end 152.4 166.37) (width 0.254) (layer F.Cu) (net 3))
 (segment (start 185.166 168.402) (end 154.432 168.402) (width 0.254) (layer F.Cu) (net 3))
 (segment (start 186.69 166.878) (end 185.166 168.402) (width 0.254) (layer F.Cu) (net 3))
 (segment (start 173.736 160.528) (end 173.228 161.036) (width 0.254) (layer F.Cu) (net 5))
 (segment (start 174.752 156.21) (end 173.736 157.226) (width 0.254) (layer F.Cu) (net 5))
 (segment (start 173.736 157.226) (end 173.736 160.528) (width 0.254) (layer F.Cu) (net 5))
 (segment (start 184.15 158.75) (end 184.15 156.972) (width 0.254) (layer F.Cu) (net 5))
 (segment (start 184.15 156.972) (end 183.388 156.21) (width 0.254) (layer F.Cu) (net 5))
 (segment (start 185.42 160.02) (end 184.15 158.75) (width 0.254) (layer F.Cu) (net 5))
 (segment (start 183.388 156.21) (end 174.752 156.21) (width 0.254) (layer F.Cu) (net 5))
 (segment (start 160.274 161.036) (end 157.48 163.83) (width 0.254) (layer F.Cu) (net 5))
 (segment (start 173.228 161.036) (end 160.274 161.036) (width 0.254) (layer F.Cu) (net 5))
 (segment (start 181.61 166.878) (end 180.848 167.64) (width 0.254) (layer F.Cu) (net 4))
 (segment (start 181.61 161.29) (end 181.61 166.624) (width 0.254) (layer F.Cu) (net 4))
 (segment (start 181.61 166.624) (end 181.61 166.878) (width 0.254) (layer F.Cu) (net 4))
 (segment (start 182.88 160.02) (end 181.61 161.29) (width 0.254) (layer F.Cu) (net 4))
 (segment (start 156.21 167.64) (end 154.94 166.37) (width 0.254) (layer F.Cu) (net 4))
 (segment (start 180.848 167.64) (end 156.21 167.64) (width 0.254) (layer F.Cu) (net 4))
 (segment (start 180.34 160.02) (end 179.07 158.75) (width 0.254) (layer F.Cu) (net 8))
 (segment (start 168.91 162.56) (end 167.64 163.83) (width 0.254) (layer F.Cu) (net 8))
 (segment (start 174.498 162.56) (end 168.91 162.56) (width 0.254) (layer F.Cu) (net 8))
 (segment (start 176.551788 160.506212) (end 174.498 162.56) (width 0.254) (layer F.Cu) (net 8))
 (segment (start 176.551788 159.490212) (end 176.551788 160.506212) (width 0.254) (layer F.Cu) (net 8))
 (segment (start 177.292 158.75) (end 176.551788 159.490212) (width 0.254) (layer F.Cu) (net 8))
 (segment (start 179.07 158.75) (end 177.292 158.75) (width 0.254) (layer F.Cu) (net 8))
 (segment (start 177.8 160.02) (end 176.53 161.29) (width 0.254) (layer F.Cu) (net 7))
 (segment (start 168.91 165.1) (end 167.64 166.37) (width 0.254) (layer F.Cu) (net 7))
 (segment (start 175.768 165.1) (end 168.91 165.1) (width 0.254) (layer F.Cu) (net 7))
 (segment (start 176.53 164.338) (end 175.768 165.1) (width 0.254) (layer F.Cu) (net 7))
 (segment (start 176.53 161.29) (end 176.53 164.338) (width 0.254) (layer F.Cu) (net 7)))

